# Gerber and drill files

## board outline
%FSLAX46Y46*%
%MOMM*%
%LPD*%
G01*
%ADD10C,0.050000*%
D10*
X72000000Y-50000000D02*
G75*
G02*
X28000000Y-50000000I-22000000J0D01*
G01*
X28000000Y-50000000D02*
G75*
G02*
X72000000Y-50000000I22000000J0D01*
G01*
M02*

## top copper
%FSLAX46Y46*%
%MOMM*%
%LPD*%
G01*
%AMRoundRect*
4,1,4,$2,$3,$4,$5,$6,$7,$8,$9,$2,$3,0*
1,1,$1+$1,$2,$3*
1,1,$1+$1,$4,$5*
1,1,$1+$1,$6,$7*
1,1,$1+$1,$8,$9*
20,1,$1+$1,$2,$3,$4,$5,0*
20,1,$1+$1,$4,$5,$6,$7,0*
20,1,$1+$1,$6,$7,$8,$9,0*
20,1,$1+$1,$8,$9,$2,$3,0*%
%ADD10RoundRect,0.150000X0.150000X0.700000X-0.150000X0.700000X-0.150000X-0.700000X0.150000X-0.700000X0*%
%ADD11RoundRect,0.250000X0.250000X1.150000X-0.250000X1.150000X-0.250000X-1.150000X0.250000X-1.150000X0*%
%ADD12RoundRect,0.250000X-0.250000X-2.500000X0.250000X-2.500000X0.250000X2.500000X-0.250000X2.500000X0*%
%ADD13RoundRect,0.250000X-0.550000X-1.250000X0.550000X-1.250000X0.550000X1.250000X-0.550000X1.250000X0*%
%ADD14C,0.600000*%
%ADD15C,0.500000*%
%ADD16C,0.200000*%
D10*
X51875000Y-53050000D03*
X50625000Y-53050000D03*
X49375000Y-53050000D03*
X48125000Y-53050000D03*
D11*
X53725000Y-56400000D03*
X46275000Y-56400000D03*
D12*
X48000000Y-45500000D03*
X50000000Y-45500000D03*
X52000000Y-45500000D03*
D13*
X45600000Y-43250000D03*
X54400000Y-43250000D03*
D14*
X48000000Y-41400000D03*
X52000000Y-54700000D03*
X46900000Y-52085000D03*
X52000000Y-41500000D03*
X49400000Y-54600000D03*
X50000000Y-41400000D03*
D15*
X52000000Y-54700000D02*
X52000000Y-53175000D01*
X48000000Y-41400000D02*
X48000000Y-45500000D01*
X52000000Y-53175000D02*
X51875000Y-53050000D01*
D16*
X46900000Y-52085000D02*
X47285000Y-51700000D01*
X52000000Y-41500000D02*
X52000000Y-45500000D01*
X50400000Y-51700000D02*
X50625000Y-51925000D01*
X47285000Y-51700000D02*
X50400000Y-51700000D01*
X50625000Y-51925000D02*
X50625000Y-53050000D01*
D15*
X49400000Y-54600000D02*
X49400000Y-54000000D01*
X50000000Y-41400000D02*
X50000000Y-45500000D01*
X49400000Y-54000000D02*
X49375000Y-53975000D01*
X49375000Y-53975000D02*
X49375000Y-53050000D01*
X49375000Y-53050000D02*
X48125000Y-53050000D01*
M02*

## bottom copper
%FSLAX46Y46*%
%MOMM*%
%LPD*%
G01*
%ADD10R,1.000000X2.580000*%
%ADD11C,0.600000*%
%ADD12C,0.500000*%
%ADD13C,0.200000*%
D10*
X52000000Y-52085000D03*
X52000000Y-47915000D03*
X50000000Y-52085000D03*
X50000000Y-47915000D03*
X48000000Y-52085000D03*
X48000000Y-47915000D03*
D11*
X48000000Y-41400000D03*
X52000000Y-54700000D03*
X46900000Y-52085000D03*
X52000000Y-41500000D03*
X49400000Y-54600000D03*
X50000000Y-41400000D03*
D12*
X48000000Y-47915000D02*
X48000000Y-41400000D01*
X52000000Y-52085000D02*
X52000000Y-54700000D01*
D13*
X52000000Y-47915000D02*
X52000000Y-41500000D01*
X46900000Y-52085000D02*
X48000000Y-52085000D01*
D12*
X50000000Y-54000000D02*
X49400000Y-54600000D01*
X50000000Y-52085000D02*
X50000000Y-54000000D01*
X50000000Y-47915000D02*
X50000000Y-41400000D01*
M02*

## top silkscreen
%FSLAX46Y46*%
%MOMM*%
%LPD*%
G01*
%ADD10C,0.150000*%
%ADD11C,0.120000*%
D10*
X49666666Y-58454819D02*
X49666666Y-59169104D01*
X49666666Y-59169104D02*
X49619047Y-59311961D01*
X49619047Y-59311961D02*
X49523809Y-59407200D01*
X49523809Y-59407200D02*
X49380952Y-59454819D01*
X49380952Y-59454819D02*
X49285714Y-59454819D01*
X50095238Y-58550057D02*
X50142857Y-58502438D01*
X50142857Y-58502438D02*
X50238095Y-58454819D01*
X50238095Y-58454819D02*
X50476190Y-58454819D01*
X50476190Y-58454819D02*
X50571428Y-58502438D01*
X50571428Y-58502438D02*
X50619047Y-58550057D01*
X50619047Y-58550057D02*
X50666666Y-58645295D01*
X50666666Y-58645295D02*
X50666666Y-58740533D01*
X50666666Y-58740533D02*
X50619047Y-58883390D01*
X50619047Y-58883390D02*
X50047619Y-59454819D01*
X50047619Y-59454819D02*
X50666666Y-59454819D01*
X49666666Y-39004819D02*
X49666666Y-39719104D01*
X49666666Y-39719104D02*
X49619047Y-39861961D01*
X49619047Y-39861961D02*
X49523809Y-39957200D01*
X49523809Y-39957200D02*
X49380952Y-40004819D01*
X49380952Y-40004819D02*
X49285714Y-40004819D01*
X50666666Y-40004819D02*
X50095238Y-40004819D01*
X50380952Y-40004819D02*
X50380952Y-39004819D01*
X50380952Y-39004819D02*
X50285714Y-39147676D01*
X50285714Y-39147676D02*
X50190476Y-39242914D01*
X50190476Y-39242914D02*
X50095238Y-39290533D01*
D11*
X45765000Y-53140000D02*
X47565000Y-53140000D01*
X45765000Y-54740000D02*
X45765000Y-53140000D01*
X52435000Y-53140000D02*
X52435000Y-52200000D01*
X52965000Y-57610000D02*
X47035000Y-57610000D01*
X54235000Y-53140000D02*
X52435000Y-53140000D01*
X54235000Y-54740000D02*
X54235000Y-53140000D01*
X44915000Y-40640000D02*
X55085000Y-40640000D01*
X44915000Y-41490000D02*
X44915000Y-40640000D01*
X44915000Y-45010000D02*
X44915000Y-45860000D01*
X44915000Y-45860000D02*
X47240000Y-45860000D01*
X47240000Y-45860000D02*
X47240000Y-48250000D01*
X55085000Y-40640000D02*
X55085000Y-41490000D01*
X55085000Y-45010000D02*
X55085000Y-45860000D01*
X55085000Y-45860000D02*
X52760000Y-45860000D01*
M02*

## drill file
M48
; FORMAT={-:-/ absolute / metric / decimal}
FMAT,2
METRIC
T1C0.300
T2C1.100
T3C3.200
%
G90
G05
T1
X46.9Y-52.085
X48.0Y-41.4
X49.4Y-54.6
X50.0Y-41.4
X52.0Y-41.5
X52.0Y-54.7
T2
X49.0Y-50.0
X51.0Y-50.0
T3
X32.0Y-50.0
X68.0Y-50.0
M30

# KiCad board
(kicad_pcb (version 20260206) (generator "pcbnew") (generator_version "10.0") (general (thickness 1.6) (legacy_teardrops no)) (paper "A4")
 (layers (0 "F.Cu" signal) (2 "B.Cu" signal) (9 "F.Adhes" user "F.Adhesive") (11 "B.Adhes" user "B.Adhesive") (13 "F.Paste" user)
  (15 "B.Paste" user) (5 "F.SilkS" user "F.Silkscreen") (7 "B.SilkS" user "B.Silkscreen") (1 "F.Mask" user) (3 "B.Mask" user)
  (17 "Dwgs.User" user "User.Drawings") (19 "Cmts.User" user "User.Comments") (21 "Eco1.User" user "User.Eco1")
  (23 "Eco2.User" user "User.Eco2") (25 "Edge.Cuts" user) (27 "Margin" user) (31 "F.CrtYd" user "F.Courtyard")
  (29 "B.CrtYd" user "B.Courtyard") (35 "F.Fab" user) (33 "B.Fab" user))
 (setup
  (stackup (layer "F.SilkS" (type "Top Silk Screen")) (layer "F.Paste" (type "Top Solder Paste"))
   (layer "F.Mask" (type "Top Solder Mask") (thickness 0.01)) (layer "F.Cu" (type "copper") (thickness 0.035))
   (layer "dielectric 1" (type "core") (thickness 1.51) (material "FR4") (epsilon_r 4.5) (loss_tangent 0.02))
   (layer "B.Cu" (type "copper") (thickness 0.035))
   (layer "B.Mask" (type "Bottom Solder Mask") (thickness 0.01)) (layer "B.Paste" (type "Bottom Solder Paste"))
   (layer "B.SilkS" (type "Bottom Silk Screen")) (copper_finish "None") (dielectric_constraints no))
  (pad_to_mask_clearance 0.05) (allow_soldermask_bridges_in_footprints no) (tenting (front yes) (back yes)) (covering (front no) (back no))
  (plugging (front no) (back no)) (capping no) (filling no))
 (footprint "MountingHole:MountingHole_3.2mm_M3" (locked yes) (layer "F.Cu") (at 32 50)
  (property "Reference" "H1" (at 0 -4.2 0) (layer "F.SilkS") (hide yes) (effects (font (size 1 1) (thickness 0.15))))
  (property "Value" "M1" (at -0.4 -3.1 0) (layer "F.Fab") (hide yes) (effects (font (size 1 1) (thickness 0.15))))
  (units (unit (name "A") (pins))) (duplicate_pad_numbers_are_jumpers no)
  (pad "" np_thru_hole circle (at 0 0) (size 3.2 3.2) (drill 3.2) (layers "*.Cu" "F.Mask")))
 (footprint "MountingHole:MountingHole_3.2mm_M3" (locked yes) (layer "F.Cu") (at 68 50)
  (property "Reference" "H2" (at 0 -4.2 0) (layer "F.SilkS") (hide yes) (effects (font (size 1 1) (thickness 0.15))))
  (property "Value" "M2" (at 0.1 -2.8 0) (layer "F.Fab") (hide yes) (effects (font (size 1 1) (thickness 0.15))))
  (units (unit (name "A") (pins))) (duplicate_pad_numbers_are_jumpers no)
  (pad "" np_thru_hole circle (at 0 0) (size 3.2 3.2) (drill 3.2) (layers "*.Cu" "F.Mask")))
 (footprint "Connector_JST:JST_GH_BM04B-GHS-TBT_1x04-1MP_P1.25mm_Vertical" (layer "F.Cu") (at 50 55 180)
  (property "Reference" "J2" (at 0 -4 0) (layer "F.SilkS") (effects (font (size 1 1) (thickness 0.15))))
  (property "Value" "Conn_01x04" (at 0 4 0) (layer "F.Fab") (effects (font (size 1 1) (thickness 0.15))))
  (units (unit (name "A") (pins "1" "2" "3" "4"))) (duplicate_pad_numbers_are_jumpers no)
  (fp_line (start 4.235 1.86) (end 2.435 1.86) (stroke (width 0.12) (type solid)) (layer "F.SilkS"))
  (fp_line (start 4.235 0.26) (end 4.235 1.86) (stroke (width 0.12) (type solid)) (layer "F.SilkS"))
  (fp_line (start -2.435 1.86) (end -2.435 2.8) (stroke (width 0.12) (type solid)) (layer "F.SilkS"))
  (fp_line (start -2.965 -2.61) (end 2.965 -2.61) (stroke (width 0.12) (type solid)) (layer "F.SilkS"))
  (fp_line (start -4.235 1.86) (end -2.435 1.86) (stroke (width 0.12) (type solid)) (layer "F.SilkS"))
  (fp_line (start -4.235 0.26) (end -4.235 1.86) (stroke (width 0.12) (type solid)) (layer "F.SilkS"))
  (pad "1" smd roundrect (at -1.875 1.95 180) (size 0.6 1.7) (layers "F.Cu" "F.Mask" "F.Paste") (roundrect_rratio 0.25) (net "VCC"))
  (pad "2" smd roundrect (at -0.625 1.95 180) (size 0.6 1.7) (layers "F.Cu" "F.Mask" "F.Paste") (roundrect_rratio 0.25) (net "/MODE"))
  (pad "3" smd roundrect (at 0.625 1.95 180) (size 0.6 1.7) (layers "F.Cu" "F.Mask" "F.Paste") (roundrect_rratio 0.25) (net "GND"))
  (pad "4" smd roundrect (at 1.875 1.95 180) (size 0.6 1.7) (layers "F.Cu" "F.Mask" "F.Paste") (roundrect_rratio 0.25) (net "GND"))
  (pad "MP" smd roundrect (at -3.725 -1.4 180) (size 1 2.8) (layers "F.Cu" "F.Mask" "F.Paste") (roundrect_rratio 0.25))
  (pad "MP" smd roundrect (at 3.725 -1.4 180) (size 1 2.8) (layers "F.Cu" "F.Mask" "F.Paste") (roundrect_rratio 0.25)))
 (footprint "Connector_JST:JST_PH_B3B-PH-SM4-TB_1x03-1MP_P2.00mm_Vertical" (layer "F.Cu") (at 50 45)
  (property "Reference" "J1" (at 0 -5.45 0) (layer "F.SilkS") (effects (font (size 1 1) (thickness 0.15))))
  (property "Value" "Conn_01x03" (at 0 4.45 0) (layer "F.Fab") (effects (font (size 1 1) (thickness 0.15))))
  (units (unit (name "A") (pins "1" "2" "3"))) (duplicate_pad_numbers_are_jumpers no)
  (fp_line (start -5.085 -4.36) (end 5.085 -4.36) (stroke (width 0.12) (type solid)) (layer "F.SilkS"))
  (fp_line (start -5.085 -3.51) (end -5.085 -4.36) (stroke (width 0.12) (type solid)) (layer "F.SilkS"))
  (fp_line (start -5.085 0.01) (end -5.085 0.86) (stroke (width 0.12) (type solid)) (layer "F.SilkS"))
  (fp_line (start -5.085 0.86) (end -2.76 0.86) (stroke (width 0.12) (type solid)) (layer "F.SilkS"))
  (fp_line (start -2.76 0.86) (end -2.76 3.25) (stroke (width 0.12) (type solid)) (layer "F.SilkS"))
  (fp_line (start 5.085 -4.36) (end 5.085 -3.51) (stroke (width 0.12) (type solid)) (layer "F.SilkS"))
  (fp_line (start 5.085 0.01) (end 5.085 0.86) (stroke (width 0.12) (type solid)) (layer "F.SilkS"))
  (fp_line (start 5.085 0.86) (end 2.76 0.86) (stroke (width 0.12) (type solid)) (layer "F.SilkS"))
  (pad "1" smd roundrect (at -2 0.5) (size 1 5.5) (layers "F.Cu" "F.Mask" "F.Paste") (roundrect_rratio 0.25) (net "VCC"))
  (pad "2" smd roundrect (at 0 0.5) (size 1 5.5) (layers "F.Cu" "F.Mask" "F.Paste") (roundrect_rratio 0.25) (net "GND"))
  (pad "3" smd roundrect (at 2 0.5) (size 1 5.5) (layers "F.Cu" "F.Mask" "F.Paste") (roundrect_rratio 0.25) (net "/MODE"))
  (pad "MP" smd roundrect (at -4.4 -1.75) (size 1.6 3) (layers "F.Cu" "F.Mask" "F.Paste") (roundrect_rratio 0.15625))
  (pad "MP" smd roundrect (at 4.4 -1.75) (size 1.6 3) (layers "F.Cu" "F.Mask" "F.Paste") (roundrect_rratio 0.15625)))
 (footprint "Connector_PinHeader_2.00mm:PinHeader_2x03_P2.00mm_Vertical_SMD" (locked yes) (layer "B.Cu") (at 50 50 90)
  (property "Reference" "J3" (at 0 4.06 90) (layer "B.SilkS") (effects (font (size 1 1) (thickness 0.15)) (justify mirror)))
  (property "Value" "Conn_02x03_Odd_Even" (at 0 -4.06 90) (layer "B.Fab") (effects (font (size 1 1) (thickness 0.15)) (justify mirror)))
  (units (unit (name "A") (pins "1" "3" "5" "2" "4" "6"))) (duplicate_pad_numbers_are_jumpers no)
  (pad "" np_thru_hole circle (at 0 -1 90) (size 0.5 0.5) (drill 1.1) (layers "*.Cu" "*.Mask"))
  (pad "" np_thru_hole circle (at 0 1 90) (size 0.5 0.5) (drill 1.1) (layers "*.Cu" "*.Mask"))
  (pad "1" smd rect (at -2.085 2 90) (size 2.58 1) (layers "B.Cu" "B.Mask" "B.Paste") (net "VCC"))
  (pad "2" smd rect (at 2.085 2 90) (size 2.58 1) (layers "B.Cu" "B.Mask" "B.Paste") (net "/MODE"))
  (pad "3" smd rect (at -2.085 0 90) (size 2.58 1) (layers "B.Cu" "B.Mask" "B.Paste") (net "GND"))
  (pad "4" smd rect (at 2.085 0 90) (size 2.58 1) (layers "B.Cu" "B.Mask" "B.Paste") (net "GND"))
  (pad "5" smd rect (at -2.085 -2 90) (size 2.58 1) (layers "B.Cu" "B.Mask" "B.Paste") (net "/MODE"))
  (pad "6" smd rect (at 2.085 -2 90) (size 2.58 1) (layers "B.Cu" "B.Mask" "B.Paste") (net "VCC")))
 (gr_circle (center 50 50) (end 72 50) (stroke (width 0.05) (type solid)) (fill no) (layer "Edge.Cuts"))
 (segment (start 52 54.7) (end 52 53.175) (width 0.5) (layer "F.Cu") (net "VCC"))
 (segment (start 48 41.4) (end 48 45.5) (width 0.5) (layer "F.Cu") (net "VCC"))
 (segment (start 52 53.175) (end 51.875 53.05) (width 0.5) (layer "F.Cu") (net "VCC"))
 (via (at 48 41.4) (size 0.6) (drill 0.3) (layers "F.Cu" "B.Cu") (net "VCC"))
 (via (at 52 54.7) (size 0.6) (drill 0.3) (layers "F.Cu" "B.Cu") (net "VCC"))
 (segment (start 48 47.915) (end 48 41.4) (width 0.5) (layer "B.Cu") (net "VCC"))
 (segment (start 52 52.085) (end 52 54.7) (width 0.5) (layer "B.Cu") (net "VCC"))
 (segment (start 46.9 52.085) (end 47.285 51.7) (width 0.2) (layer "F.Cu") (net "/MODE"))
 (segment (start 52 41.5) (end 52 45.5) (width 0.2) (layer "F.Cu") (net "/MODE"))
 (segment (start 50.4 51.7) (end 50.625 51.925) (width 0.2) (layer "F.Cu") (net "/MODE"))
 (segment (start 47.285 51.7) (end 50.4 51.7) (width 0.2) (layer "F.Cu") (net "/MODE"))
 (segment (start 50.625 51.925) (end 50.625 53.05) (width 0.2) (layer "F.Cu") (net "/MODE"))
 (via (at 46.9 52.085) (size 0.6) (drill 0.3) (layers "F.Cu" "B.Cu") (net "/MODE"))
 (via (at 52 41.5) (size 0.6) (drill 0.3) (layers "F.Cu" "B.Cu") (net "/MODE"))
 (segment (start 52 47.915) (end 52 41.5) (width 0.2) (layer "B.Cu") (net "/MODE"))
 (segment (start 46.9 52.085) (end 48 52.085) (width 0.2) (layer "B.Cu") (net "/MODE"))
 (segment (start 49.4 54.6) (end 49.4 54) (width 0.5) (layer "F.Cu") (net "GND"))
 (segment (start 50 41.4) (end 50 45.5) (width 0.5) (layer "F.Cu") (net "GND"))
 (segment (start 49.4 54) (end 49.375 53.975) (width 0.5) (layer "F.Cu") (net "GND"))
 (segment (start 49.375 53.975) (end 49.375 53.05) (width 0.5) (layer "F.Cu") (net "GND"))
 (segment (start 49.375 53.05) (end 48.125 53.05) (width 0.5) (layer "F.Cu") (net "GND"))
 (via (at 49.4 54.6) (size 0.6) (drill 0.3) (layers "F.Cu" "B.Cu") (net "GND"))
 (via (at 50 41.4) (size 0.6) (drill 0.3) (layers "F.Cu" "B.Cu") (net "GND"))
 (segment (start 50 54) (end 49.4 54.6) (width 0.5) (layer "B.Cu") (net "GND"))
 (segment (start 50 52.085) (end 50 54) (width 0.5) (layer "B.Cu") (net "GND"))
 (segment (start 50 47.915) (end 50 41.4) (width 0.5) (layer "B.Cu") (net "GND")))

